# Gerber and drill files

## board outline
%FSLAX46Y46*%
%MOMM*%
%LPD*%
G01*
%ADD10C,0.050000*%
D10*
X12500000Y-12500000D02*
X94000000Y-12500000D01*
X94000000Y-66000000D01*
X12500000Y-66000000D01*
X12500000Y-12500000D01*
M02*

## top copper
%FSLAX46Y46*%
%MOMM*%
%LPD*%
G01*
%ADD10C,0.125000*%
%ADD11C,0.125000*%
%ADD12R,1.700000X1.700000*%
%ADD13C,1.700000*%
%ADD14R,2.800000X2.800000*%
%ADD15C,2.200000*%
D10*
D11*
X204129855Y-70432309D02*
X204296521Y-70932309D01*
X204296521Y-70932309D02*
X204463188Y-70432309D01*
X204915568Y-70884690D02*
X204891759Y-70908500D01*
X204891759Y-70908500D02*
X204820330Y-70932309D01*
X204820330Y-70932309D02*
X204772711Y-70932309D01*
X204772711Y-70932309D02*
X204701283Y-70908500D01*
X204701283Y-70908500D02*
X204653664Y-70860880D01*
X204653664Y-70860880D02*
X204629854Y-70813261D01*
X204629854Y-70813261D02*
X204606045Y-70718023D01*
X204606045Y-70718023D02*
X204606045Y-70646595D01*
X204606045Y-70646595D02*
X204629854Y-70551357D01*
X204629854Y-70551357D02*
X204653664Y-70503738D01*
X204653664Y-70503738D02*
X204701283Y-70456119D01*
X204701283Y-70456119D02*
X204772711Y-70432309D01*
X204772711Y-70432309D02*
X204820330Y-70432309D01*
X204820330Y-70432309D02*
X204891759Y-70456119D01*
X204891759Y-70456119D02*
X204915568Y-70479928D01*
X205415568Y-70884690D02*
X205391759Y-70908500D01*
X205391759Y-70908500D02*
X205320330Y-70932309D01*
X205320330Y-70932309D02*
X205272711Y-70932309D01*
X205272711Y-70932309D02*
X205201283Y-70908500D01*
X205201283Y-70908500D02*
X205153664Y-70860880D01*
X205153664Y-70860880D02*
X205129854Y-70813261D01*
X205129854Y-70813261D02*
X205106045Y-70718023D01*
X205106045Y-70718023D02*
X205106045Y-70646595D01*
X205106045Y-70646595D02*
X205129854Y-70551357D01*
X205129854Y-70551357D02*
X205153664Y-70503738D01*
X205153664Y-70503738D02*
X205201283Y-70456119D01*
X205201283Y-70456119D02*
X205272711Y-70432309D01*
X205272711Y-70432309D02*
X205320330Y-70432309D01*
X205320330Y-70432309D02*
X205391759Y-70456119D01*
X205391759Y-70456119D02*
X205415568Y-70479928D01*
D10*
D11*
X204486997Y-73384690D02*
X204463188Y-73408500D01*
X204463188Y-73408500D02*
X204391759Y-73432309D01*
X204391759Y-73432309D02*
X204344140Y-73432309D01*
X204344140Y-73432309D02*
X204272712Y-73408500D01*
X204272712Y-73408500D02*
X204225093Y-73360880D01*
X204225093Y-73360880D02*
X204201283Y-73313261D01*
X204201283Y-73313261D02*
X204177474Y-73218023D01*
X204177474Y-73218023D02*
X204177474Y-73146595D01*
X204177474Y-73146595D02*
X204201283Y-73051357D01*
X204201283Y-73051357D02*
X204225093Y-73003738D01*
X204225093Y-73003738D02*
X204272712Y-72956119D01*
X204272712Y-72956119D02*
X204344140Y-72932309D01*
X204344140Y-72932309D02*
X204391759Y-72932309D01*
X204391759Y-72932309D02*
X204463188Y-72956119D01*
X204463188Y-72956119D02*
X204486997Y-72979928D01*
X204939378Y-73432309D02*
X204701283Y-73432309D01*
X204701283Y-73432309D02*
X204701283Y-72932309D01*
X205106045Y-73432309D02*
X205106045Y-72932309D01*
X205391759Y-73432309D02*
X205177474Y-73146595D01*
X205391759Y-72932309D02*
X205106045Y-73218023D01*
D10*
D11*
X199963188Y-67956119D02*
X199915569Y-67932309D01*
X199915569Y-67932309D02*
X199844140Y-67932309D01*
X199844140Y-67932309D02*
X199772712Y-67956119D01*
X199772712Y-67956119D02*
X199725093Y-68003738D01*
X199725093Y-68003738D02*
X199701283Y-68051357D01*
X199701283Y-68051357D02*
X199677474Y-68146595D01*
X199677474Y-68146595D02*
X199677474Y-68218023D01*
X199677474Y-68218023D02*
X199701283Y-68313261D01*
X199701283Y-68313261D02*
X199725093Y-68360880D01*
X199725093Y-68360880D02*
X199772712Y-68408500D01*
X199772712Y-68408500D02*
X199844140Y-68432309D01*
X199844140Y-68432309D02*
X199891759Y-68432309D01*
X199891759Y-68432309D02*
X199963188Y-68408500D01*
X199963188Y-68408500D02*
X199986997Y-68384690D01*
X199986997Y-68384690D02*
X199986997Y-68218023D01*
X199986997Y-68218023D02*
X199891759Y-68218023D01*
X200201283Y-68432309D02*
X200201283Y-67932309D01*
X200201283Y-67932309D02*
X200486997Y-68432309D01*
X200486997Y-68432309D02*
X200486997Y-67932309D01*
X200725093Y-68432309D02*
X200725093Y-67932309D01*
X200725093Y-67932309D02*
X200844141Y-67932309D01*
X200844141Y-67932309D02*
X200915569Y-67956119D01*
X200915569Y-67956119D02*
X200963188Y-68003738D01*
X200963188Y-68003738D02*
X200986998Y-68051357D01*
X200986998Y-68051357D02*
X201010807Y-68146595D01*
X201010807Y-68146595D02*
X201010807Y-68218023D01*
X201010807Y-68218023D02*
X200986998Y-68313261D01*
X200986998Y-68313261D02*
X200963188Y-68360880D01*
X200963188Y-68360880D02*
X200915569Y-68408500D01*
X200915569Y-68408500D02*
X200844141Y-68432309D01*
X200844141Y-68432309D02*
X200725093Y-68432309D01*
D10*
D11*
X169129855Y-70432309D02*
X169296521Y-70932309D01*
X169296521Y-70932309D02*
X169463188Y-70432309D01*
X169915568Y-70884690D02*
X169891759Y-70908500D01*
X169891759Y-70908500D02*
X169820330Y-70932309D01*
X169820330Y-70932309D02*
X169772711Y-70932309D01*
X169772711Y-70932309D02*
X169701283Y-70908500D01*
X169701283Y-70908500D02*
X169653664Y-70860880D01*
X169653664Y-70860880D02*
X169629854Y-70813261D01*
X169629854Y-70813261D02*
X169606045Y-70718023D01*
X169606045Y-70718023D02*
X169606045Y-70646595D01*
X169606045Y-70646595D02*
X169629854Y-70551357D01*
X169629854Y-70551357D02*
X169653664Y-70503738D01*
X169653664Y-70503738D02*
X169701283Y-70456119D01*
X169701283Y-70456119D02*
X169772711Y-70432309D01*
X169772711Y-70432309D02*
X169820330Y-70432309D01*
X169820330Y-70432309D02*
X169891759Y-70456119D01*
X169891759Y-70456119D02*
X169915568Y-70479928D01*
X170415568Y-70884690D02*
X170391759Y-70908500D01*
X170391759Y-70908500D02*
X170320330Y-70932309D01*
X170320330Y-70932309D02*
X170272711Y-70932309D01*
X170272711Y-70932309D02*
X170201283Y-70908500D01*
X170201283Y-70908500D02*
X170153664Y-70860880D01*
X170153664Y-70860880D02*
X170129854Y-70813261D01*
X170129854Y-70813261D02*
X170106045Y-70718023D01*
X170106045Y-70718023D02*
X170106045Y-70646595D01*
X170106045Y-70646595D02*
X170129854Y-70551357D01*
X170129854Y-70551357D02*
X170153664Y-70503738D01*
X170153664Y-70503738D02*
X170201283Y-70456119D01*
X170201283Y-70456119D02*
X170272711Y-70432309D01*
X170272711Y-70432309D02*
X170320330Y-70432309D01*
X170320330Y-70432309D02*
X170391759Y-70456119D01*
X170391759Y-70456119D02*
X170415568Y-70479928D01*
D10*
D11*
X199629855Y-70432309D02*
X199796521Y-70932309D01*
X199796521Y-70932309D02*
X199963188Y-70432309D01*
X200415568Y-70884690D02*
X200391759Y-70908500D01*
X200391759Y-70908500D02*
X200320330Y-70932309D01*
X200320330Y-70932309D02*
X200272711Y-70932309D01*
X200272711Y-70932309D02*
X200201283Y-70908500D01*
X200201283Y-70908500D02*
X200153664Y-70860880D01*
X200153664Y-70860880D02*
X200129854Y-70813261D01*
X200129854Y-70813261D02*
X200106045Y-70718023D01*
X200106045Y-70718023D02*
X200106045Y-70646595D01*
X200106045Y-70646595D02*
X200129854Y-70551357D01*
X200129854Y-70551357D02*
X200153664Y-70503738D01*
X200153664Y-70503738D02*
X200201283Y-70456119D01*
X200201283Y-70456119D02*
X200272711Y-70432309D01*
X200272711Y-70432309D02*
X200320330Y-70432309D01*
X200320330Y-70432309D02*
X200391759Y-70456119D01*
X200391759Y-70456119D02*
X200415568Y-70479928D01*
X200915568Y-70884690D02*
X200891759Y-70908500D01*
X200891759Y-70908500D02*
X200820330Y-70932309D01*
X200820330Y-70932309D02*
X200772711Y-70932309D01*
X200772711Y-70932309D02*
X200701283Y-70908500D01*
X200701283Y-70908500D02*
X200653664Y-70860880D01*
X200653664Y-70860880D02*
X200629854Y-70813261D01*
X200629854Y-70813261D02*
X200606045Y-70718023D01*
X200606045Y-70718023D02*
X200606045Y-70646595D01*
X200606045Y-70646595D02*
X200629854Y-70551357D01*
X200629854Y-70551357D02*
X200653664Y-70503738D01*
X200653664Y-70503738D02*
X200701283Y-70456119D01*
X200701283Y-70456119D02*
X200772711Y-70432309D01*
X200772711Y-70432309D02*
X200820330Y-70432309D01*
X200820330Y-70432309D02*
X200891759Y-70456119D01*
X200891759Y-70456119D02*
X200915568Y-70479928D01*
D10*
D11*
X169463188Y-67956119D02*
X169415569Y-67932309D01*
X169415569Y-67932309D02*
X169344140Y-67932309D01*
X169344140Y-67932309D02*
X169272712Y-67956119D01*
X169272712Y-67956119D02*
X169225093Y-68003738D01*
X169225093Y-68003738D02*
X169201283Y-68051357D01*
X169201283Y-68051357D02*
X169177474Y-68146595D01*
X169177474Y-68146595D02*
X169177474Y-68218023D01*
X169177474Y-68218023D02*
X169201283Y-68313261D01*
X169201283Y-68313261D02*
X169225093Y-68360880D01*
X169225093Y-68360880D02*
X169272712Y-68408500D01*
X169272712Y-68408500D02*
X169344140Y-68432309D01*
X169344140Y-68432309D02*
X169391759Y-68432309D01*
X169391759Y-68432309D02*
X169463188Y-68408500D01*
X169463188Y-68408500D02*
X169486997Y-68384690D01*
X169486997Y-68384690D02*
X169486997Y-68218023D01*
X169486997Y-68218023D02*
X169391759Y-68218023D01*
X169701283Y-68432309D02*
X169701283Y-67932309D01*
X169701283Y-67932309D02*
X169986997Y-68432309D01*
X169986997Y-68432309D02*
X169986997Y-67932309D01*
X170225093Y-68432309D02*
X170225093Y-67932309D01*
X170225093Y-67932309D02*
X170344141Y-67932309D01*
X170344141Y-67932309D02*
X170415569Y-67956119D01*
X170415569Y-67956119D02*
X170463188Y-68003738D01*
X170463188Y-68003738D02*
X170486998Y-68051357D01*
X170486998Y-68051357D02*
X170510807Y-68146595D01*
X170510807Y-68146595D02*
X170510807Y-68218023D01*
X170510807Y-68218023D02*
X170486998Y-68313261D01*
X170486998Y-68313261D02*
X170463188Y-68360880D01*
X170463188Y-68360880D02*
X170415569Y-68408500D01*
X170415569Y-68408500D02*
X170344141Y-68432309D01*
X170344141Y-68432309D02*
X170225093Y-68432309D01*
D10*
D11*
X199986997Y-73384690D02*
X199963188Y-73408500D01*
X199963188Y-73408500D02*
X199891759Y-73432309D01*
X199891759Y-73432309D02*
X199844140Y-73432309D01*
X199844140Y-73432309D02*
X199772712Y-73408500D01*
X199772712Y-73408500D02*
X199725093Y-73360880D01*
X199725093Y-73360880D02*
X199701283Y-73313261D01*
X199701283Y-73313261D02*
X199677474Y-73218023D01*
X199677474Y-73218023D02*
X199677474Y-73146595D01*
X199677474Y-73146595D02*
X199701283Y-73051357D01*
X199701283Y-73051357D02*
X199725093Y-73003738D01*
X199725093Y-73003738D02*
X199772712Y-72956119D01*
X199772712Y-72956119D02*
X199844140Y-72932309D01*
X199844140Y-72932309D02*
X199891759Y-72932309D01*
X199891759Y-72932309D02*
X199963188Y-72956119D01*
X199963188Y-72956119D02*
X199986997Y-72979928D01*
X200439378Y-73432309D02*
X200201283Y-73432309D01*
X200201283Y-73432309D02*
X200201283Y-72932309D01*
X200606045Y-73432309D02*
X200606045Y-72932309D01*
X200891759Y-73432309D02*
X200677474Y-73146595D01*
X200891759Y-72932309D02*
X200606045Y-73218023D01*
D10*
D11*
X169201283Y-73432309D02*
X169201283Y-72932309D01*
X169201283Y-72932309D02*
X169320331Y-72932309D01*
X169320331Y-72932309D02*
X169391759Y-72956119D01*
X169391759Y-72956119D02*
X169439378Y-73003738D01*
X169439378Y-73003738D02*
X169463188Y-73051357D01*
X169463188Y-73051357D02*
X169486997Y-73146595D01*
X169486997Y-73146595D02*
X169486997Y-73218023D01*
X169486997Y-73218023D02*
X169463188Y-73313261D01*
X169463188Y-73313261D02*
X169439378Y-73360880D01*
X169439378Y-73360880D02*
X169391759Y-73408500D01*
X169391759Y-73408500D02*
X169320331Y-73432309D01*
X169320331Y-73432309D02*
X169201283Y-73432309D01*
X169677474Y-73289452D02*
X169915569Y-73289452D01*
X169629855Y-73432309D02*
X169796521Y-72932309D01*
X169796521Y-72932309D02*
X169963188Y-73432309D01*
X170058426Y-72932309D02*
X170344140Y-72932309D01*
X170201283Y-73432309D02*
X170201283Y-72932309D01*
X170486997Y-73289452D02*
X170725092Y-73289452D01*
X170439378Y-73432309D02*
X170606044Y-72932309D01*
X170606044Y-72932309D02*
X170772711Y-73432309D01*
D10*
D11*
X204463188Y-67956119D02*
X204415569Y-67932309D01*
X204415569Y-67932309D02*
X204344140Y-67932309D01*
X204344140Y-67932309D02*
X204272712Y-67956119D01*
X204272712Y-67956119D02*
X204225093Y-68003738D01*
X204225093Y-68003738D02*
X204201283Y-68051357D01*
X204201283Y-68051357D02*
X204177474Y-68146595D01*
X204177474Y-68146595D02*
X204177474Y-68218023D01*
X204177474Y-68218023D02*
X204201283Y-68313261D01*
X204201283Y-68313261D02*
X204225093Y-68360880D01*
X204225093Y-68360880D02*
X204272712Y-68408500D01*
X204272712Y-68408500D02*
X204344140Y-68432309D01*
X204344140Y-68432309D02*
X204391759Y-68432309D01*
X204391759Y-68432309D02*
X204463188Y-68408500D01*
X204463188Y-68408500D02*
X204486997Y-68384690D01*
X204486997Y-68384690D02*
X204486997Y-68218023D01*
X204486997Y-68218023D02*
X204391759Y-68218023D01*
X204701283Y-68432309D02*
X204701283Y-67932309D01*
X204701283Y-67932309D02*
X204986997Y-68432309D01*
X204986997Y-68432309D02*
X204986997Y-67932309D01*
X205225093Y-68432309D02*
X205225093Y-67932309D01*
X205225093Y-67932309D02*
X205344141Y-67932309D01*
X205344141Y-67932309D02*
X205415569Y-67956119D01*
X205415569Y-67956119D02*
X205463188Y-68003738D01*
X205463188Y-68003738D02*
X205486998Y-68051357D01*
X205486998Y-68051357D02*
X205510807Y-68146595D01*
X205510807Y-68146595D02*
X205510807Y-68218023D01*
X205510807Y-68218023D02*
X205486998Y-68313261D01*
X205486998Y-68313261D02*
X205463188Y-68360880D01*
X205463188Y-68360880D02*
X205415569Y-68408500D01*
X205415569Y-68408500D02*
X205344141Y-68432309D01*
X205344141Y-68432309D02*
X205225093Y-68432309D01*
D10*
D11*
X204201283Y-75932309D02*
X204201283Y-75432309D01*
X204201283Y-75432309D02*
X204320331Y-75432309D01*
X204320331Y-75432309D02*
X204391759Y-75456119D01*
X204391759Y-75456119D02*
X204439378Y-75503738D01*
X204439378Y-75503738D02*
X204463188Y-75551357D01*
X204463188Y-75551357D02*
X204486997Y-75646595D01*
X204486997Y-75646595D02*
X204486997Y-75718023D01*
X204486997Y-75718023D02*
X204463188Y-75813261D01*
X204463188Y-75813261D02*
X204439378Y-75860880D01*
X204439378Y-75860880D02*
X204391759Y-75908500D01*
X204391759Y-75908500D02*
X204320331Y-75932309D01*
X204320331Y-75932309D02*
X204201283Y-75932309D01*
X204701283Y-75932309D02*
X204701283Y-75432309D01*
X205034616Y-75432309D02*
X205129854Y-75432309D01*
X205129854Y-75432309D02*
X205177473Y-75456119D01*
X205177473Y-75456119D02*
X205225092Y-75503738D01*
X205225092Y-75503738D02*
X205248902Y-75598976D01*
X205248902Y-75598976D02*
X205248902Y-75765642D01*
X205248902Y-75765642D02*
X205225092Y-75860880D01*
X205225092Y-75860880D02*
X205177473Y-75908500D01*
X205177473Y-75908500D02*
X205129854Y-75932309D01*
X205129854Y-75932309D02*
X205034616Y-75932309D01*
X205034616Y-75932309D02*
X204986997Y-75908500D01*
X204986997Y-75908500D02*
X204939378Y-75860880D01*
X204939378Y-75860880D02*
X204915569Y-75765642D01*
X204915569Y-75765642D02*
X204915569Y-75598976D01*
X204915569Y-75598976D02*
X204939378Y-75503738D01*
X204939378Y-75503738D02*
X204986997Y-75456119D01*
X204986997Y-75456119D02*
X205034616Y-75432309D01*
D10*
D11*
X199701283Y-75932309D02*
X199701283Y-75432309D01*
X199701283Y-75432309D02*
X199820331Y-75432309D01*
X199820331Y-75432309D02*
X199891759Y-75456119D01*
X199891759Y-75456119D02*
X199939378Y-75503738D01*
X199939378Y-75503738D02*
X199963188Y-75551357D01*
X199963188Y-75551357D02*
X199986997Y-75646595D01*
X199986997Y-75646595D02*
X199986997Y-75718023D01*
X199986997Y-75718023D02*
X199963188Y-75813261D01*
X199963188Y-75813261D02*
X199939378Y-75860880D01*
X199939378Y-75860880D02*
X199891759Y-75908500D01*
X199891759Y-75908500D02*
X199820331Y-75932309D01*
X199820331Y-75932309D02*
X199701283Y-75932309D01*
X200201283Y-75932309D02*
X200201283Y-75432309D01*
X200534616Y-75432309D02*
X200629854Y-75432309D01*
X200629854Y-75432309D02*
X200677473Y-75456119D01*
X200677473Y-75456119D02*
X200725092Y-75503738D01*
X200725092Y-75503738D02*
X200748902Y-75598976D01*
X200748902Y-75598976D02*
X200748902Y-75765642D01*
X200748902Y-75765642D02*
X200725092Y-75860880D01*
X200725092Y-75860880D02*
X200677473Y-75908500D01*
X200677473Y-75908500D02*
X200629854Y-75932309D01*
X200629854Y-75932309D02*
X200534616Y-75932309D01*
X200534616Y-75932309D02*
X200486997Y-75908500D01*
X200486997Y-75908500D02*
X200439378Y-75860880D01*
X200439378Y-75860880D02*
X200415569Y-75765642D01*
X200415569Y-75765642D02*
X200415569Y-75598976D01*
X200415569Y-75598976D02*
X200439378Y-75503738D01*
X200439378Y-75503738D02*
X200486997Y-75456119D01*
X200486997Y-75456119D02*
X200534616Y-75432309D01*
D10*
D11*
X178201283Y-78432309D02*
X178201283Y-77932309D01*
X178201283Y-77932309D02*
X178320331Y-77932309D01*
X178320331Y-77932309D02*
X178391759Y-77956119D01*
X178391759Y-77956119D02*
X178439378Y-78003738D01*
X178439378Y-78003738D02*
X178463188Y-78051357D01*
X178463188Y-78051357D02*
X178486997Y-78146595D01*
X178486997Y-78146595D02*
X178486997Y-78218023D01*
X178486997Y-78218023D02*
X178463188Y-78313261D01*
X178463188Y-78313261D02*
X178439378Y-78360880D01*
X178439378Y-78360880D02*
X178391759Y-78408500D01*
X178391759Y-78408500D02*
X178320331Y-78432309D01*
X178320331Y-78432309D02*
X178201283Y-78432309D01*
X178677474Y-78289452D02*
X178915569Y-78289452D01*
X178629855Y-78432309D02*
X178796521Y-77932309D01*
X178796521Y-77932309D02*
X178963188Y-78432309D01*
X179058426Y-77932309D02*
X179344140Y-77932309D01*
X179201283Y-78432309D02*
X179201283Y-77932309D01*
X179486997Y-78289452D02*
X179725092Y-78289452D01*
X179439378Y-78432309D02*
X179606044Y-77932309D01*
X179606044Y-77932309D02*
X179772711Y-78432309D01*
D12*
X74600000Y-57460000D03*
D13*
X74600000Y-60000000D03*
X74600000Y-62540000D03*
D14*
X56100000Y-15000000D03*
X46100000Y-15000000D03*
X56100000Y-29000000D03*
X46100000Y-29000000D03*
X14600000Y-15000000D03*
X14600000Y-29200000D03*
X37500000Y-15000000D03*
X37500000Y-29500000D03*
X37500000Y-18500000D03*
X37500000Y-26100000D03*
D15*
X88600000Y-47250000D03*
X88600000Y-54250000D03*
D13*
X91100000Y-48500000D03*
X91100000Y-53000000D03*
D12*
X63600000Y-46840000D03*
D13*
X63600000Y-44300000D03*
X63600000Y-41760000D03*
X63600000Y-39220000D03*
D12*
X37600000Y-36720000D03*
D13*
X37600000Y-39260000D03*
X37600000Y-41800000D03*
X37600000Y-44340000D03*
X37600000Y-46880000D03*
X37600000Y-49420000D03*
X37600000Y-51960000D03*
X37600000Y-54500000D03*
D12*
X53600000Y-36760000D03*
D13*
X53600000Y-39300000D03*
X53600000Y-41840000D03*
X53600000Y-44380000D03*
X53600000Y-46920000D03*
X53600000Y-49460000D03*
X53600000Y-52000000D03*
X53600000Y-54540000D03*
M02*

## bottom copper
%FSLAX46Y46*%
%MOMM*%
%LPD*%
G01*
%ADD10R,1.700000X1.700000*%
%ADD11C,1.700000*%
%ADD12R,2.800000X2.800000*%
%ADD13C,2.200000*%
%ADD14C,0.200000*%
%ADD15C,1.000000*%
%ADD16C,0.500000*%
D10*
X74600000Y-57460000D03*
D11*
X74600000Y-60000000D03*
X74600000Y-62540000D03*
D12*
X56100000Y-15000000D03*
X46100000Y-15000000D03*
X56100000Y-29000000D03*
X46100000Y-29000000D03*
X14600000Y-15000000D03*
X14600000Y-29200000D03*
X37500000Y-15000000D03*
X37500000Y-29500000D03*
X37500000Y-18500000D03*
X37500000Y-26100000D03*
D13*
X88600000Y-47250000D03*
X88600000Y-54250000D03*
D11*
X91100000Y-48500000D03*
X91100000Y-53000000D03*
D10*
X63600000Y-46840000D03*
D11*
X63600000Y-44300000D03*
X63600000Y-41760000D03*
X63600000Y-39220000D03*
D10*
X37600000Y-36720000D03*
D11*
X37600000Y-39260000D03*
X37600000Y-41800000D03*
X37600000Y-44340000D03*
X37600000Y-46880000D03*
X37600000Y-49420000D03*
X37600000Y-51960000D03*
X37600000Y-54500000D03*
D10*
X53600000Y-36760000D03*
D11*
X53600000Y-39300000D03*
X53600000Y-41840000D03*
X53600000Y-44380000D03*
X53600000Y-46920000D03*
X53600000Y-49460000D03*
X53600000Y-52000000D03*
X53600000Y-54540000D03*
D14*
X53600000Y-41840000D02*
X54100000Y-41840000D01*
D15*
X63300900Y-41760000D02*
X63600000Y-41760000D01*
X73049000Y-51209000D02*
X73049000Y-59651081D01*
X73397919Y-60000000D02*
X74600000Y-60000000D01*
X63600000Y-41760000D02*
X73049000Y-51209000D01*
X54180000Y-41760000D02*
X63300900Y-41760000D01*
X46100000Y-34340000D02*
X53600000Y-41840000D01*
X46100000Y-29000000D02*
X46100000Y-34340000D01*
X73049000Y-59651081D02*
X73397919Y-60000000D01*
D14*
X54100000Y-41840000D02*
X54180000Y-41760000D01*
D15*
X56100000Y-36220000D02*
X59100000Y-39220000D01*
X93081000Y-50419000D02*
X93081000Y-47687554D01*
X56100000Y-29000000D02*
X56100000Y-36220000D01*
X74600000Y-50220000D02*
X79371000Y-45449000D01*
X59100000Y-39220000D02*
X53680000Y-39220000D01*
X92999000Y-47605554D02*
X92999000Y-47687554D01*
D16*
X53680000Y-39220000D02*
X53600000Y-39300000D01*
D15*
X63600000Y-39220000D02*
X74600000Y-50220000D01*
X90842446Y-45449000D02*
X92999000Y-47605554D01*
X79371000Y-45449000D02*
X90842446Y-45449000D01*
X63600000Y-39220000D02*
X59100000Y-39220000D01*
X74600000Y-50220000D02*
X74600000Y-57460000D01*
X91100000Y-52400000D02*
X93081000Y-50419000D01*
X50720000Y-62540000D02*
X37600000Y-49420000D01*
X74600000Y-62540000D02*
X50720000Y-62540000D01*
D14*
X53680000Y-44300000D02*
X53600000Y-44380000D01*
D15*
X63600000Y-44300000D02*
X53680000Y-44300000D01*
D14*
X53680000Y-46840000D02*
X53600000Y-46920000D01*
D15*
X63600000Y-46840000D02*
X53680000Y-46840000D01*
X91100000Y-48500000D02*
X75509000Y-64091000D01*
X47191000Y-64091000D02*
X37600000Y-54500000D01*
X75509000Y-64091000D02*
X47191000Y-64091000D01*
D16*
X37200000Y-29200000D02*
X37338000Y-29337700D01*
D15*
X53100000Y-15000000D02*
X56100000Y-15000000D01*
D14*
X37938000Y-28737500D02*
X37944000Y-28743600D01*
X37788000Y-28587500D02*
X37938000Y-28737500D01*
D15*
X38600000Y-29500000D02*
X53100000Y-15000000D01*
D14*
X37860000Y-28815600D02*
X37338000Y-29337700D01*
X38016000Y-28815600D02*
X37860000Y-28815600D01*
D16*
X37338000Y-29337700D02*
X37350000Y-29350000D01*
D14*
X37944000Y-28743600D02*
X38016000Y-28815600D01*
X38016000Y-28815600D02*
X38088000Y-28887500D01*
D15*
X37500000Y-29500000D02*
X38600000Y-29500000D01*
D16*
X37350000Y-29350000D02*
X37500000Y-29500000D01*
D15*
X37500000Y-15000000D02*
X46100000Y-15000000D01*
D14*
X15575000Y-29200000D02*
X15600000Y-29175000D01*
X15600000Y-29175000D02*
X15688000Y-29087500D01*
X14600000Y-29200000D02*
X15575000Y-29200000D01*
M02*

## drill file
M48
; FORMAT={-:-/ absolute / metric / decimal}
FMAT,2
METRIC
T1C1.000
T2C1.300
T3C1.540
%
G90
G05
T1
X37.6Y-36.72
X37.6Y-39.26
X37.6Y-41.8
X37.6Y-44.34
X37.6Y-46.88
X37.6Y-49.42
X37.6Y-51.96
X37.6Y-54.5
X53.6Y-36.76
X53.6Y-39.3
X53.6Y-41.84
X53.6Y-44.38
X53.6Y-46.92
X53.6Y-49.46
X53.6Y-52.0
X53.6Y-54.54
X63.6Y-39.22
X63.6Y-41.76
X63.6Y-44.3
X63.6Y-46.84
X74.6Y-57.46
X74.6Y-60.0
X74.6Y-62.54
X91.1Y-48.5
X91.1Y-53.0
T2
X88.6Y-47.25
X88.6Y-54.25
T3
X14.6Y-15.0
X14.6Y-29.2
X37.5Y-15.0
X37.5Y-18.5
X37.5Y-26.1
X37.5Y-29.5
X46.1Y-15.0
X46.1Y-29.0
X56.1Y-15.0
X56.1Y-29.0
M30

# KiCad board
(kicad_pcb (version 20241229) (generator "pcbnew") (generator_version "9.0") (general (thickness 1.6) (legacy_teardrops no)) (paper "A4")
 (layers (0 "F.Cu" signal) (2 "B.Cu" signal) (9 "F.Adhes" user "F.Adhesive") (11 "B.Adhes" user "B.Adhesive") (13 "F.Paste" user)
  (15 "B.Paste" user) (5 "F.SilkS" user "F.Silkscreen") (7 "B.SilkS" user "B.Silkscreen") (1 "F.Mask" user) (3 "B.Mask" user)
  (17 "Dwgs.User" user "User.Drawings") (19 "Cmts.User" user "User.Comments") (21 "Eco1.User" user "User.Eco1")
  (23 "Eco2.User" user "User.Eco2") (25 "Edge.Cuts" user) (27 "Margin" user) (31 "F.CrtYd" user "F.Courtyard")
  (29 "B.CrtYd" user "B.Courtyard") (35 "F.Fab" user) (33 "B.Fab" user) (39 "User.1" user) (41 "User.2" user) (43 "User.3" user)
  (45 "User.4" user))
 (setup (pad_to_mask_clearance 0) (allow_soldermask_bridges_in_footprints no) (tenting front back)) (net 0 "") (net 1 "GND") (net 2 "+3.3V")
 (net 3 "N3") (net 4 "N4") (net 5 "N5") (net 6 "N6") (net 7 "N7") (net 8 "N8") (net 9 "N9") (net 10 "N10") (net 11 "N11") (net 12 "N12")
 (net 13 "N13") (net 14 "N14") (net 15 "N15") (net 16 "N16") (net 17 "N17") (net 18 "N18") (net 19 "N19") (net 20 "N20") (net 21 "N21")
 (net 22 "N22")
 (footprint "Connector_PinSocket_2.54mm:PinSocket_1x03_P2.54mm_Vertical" (layer "F.Cu") (at 74.6 57.46)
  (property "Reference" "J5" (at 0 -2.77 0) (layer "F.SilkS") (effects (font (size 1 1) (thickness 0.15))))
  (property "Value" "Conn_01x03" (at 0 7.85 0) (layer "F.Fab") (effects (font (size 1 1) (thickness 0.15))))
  (pad "1" thru_hole rect (at 0 0) (size 1.7 1.7) (drill 1) (layers "*.Cu" "*.Mask") (remove_unused_layers no) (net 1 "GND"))
  (pad "2" thru_hole circle (at 0 2.54) (size 1.7 1.7) (drill 1) (layers "*.Cu" "*.Mask") (remove_unused_layers no) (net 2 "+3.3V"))
  (pad "3" thru_hole circle (at 0 5.08) (size 1.7 1.7) (drill 1) (layers "*.Cu" "*.Mask") (remove_unused_layers no) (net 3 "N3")))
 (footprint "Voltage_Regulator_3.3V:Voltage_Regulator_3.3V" (layer "F.Cu") (at 57.6 13.5 -90)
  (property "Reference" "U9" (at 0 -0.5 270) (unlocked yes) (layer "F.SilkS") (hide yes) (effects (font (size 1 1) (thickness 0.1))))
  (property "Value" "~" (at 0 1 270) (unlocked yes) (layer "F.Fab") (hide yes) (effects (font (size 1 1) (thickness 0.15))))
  (pad "1" thru_hole rect (at 1.5 1.5 180) (size 2.8 2.8) (drill 1.54) (layers "*.Cu" "*.Mask") (remove_unused_layers no) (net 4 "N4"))
  (pad "2" thru_hole rect (at 1.5 11.5 180) (size 2.8 2.8) (drill 1.54) (layers "*.Cu" "*.Mask") (remove_unused_layers no) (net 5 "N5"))
  (pad "3" thru_hole rect (at 15.5 1.5 180) (size 2.8 2.8) (drill 1.54) (layers "*.Cu" "*.Mask") (remove_unused_layers no) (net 1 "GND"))
  (pad "4" thru_hole rect (at 15.5 11.5 180) (size 2.8 2.8) (drill 1.54) (layers "*.Cu" "*.Mask") (remove_unused_layers no) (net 2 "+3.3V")))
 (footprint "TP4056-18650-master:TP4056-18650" (layer "F.Cu") (at 12.9 13.3)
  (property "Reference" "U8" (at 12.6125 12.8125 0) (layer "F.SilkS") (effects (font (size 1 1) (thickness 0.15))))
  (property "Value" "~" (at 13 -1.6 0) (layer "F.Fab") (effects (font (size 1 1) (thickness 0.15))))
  (pad "1" thru_hole rect (at 1.7 1.7) (size 2.8 2.8) (drill 1.54) (layers "*.Cu" "*.Mask") (remove_unused_layers no) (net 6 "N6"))
  (pad "2" thru_hole rect (at 1.7 15.9) (size 2.8 2.8) (drill 1.54) (layers "*.Cu" "*.Mask") (remove_unused_layers no) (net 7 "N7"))
  (pad "3" thru_hole rect (at 24.6 1.7) (size 2.8 2.8) (drill 1.54) (layers "*.Cu" "*.Mask") (remove_unused_layers no) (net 5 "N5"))
  (pad "4" thru_hole rect (at 24.6 16.2) (size 2.8 2.8) (drill 1.54) (layers "*.Cu" "*.Mask") (remove_unused_layers no) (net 4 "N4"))
  (pad "5" thru_hole rect (at 24.6 5.2) (size 2.8 2.8) (drill 1.54) (layers "*.Cu" "*.Mask") (remove_unused_layers no) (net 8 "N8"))
  (pad "6" thru_hole rect (at 24.6 12.8) (size 2.8 2.8) (drill 1.54) (layers "*.Cu" "*.Mask") (remove_unused_layers no) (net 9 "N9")))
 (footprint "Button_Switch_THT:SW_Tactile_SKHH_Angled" (layer "F.Cu") (at 91.1 48.5 -90)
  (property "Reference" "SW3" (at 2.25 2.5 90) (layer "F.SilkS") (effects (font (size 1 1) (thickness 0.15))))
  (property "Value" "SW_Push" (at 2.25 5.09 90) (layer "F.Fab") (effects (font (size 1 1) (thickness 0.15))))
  (pad "" thru_hole circle (at -1.25 2.5 90) (size 2.2 2.2) (drill 1.3) (layers "*.Cu" "*.Mask") (remove_unused_layers no))
  (pad "" thru_hole circle (at 5.75 2.5 90) (size 2.2 2.2) (drill 1.3) (layers "*.Cu" "*.Mask") (remove_unused_layers no))
  (pad "1" thru_hole circle (at 0 0 90) (size 1.7 1.7) (drill 1) (layers "*.Cu" "*.Mask") (remove_unused_layers no) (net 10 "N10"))
  (pad "2" thru_hole circle (at 4.5 0 90) (size 1.7 1.7) (drill 1) (layers "*.Cu" "*.Mask") (remove_unused_layers no) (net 1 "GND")))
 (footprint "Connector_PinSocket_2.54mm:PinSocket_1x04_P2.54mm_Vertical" (layer "F.Cu") (at 63.6 46.84 180)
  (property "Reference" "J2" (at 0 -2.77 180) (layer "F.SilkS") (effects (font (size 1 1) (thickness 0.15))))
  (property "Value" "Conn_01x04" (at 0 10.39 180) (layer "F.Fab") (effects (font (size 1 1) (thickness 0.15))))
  (pad "1" thru_hole rect (at 0 0 180) (size 1.7 1.7) (drill 1) (layers "*.Cu" "*.Mask") (remove_unused_layers no) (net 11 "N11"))
  (pad "2" thru_hole circle (at 0 2.54 180) (size 1.7 1.7) (drill 1) (layers "*.Cu" "*.Mask") (remove_unused_layers no) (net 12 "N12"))
  (pad "3" thru_hole circle (at 0 5.08 180) (size 1.7 1.7) (drill 1) (layers "*.Cu" "*.Mask") (remove_unused_layers no) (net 2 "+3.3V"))
  (pad "4" thru_hole circle (at 0 7.62 180) (size 1.7 1.7) (drill 1) (layers "*.Cu" "*.Mask") (remove_unused_layers no) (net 1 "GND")))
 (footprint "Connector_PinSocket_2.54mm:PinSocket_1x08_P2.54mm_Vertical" (layer "F.Cu") (at 37.6 36.72)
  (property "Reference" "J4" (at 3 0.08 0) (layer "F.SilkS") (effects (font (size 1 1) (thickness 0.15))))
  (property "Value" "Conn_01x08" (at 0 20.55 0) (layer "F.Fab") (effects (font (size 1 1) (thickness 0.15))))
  (pad "1" thru_hole rect (at 0 0) (size 1.7 1.7) (drill 1) (layers "*.Cu" "*.Mask") (remove_unused_layers no) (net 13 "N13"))
  (pad "2" thru_hole circle (at 0 2.54) (size 1.7 1.7) (drill 1) (layers "*.Cu" "*.Mask") (remove_unused_layers no) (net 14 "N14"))
  (pad "3" thru_hole circle (at 0 5.08) (size 1.7 1.7) (drill 1) (layers "*.Cu" "*.Mask") (remove_unused_layers no) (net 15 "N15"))
  (pad "4" thru_hole circle (at 0 7.62) (size 1.7 1.7) (drill 1) (layers "*.Cu" "*.Mask") (remove_unused_layers no) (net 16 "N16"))
  (pad "5" thru_hole circle (at 0 10.16) (size 1.7 1.7) (drill 1) (layers "*.Cu" "*.Mask") (remove_unused_layers no) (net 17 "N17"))
  (pad "6" thru_hole circle (at 0 12.7) (size 1.7 1.7) (drill 1) (layers "*.Cu" "*.Mask") (remove_unused_layers no) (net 3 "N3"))
  (pad "7" thru_hole circle (at 0 15.24) (size 1.7 1.7) (drill 1) (layers "*.Cu" "*.Mask") (remove_unused_layers no) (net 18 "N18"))
  (pad "8" thru_hole circle (at 0 17.78) (size 1.7 1.7) (drill 1) (layers "*.Cu" "*.Mask") (remove_unused_layers no) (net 10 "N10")))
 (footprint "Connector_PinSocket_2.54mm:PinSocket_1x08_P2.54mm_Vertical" (layer "F.Cu") (at 53.6 36.76)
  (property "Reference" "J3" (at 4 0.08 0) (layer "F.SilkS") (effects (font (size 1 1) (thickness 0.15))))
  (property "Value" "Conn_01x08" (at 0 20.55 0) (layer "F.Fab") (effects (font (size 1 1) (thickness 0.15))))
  (pad "1" thru_hole rect (at 0 0) (size 1.7 1.7) (drill 1) (layers "*.Cu" "*.Mask") (remove_unused_layers no) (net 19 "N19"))
  (pad "2" thru_hole circle (at 0 2.54) (size 1.7 1.7) (drill 1) (layers "*.Cu" "*.Mask") (remove_unused_layers no) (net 1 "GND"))
  (pad "3" thru_hole circle (at 0 5.08) (size 1.7 1.7) (drill 1) (layers "*.Cu" "*.Mask") (remove_unused_layers no) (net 2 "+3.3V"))
  (pad "4" thru_hole circle (at 0 7.62) (size 1.7 1.7) (drill 1) (layers "*.Cu" "*.Mask") (remove_unused_layers no) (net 12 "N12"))
  (pad "5" thru_hole circle (at 0 10.16) (size 1.7 1.7) (drill 1) (layers "*.Cu" "*.Mask") (remove_unused_layers no) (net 11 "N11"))
  (pad "6" thru_hole circle (at 0 12.7) (size 1.7 1.7) (drill 1) (layers "*.Cu" "*.Mask") (remove_unused_layers no) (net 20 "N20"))
  (pad "7" thru_hole circle (at 0 15.24) (size 1.7 1.7) (drill 1) (layers "*.Cu" "*.Mask") (remove_unused_layers no) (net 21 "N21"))
  (pad "8" thru_hole circle (at 0 17.78) (size 1.7 1.7) (drill 1) (layers "*.Cu" "*.Mask") (remove_unused_layers no) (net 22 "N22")))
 (gr_rect (start 12.5 12.5) (end 94 66) (stroke (width 0.05) (type default)) (fill no) (layer "Edge.Cuts"))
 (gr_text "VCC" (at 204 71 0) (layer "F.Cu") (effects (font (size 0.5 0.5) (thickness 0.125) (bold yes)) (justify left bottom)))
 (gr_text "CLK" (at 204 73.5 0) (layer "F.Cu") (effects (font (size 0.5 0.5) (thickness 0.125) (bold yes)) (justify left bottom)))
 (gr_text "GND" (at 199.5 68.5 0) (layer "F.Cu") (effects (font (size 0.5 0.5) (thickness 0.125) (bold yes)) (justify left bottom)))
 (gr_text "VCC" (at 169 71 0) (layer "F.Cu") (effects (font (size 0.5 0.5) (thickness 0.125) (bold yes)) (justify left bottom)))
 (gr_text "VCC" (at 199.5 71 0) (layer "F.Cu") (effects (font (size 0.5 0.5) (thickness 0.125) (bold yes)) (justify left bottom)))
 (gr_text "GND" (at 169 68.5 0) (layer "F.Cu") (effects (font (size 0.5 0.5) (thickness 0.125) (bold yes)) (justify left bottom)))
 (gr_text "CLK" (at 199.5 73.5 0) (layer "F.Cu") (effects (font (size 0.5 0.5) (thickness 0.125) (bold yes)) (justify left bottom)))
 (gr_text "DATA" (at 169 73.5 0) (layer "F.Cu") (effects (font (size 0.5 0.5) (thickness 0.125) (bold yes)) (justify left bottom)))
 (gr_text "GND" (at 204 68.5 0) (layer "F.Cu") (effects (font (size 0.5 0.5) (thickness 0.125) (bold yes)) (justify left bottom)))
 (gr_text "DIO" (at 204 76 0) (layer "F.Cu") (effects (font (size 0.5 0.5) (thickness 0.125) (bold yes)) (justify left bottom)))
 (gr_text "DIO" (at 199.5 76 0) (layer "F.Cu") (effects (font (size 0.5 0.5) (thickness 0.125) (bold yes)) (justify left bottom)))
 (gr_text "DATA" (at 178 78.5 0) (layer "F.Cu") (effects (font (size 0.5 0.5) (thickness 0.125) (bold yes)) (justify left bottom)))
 (segment (start 53.6 41.84) (end 54.1 41.84) (width 0.2) (layer "B.Cu") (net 2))
 (segment (start 63.3009 41.76) (end 63.6 41.76) (width 1) (layer "B.Cu") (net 2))
 (segment (start 73.049 51.209) (end 73.049 59.651081) (width 1) (layer "B.Cu") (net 2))
 (segment (start 73.397919 60) (end 74.6 60) (width 1) (layer "B.Cu") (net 2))
 (segment (start 63.6 41.76) (end 73.049 51.209) (width 1) (layer "B.Cu") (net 2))
 (segment (start 54.18 41.76) (end 63.3009 41.76) (width 1) (layer "B.Cu") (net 2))
 (segment (start 46.1 34.34) (end 53.6 41.84) (width 1) (layer "B.Cu") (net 2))
 (segment (start 46.1 29) (end 46.1 34.34) (width 1) (layer "B.Cu") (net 2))
 (segment (start 73.049 59.651081) (end 73.397919 60) (width 1) (layer "B.Cu") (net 2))
 (segment (start 54.1 41.84) (end 54.18 41.76) (width 0.2) (layer "B.Cu") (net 2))
 (segment (start 56.1 36.22) (end 59.1 39.22) (width 1) (layer "B.Cu") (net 1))
 (segment (start 93.081 50.419) (end 93.081 47.687554) (width 1) (layer "B.Cu") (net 1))
 (segment (start 56.1 29) (end 56.1 36.22) (width 1) (layer "B.Cu") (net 1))
 (segment (start 74.6 50.22) (end 79.371 45.449) (width 1) (layer "B.Cu") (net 1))
 (segment (start 59.1 39.22) (end 53.68 39.22) (width 1) (layer "B.Cu") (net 1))
 (segment (start 92.999 47.605554) (end 92.999 47.687554) (width 1) (layer "B.Cu") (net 1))
 (segment (start 53.68 39.22) (end 53.6 39.3) (width 0.5) (layer "B.Cu") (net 1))
 (segment (start 63.6 39.22) (end 74.6 50.22) (width 1) (layer "B.Cu") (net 1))
 (segment (start 90.842446 45.449) (end 92.999 47.605554) (width 1) (layer "B.Cu") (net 1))
 (segment (start 79.371 45.449) (end 90.842446 45.449) (width 1) (layer "B.Cu") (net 1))
 (segment (start 63.6 39.22) (end 59.1 39.22) (width 1) (layer "B.Cu") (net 1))
 (segment (start 74.6 50.22) (end 74.6 57.46) (width 1) (layer "B.Cu") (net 1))
 (segment (start 91.1 52.4) (end 93.081 50.419) (width 1) (layer "B.Cu") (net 1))
 (segment (start 50.72 62.54) (end 37.6 49.42) (width 1) (layer "B.Cu") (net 3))
 (segment (start 74.6 62.54) (end 50.72 62.54) (width 1) (layer "B.Cu") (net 3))
 (segment (start 53.68 44.3) (end 53.6 44.38) (width 0.2) (layer "B.Cu") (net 12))
 (segment (start 63.6 44.3) (end 53.68 44.3) (width 1) (layer "B.Cu") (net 12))
 (segment (start 53.68 46.84) (end 53.6 46.92) (width 0.2) (layer "B.Cu") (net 11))
 (segment (start 63.6 46.84) (end 53.68 46.84) (width 1) (layer "B.Cu") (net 11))
 (segment (start 91.1 48.5) (end 75.509 64.091) (width 1) (layer "B.Cu") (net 10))
 (segment (start 47.191 64.091) (end 37.6 54.5) (width 1) (layer "B.Cu") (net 10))
 (segment (start 75.509 64.091) (end 47.191 64.091) (width 1) (layer "B.Cu") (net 10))
 (segment (start 37.2 29.2) (end 37.338 29.3377) (width 0.5) (layer "B.Cu") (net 4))
 (segment (start 53.1 15) (end 56.1 15) (width 1) (layer "B.Cu") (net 4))
 (segment (start 37.938 28.7375) (end 37.944 28.7436) (width 0.2) (layer "B.Cu") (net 4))
 (segment (start 37.788 28.5875) (end 37.938 28.7375) (width 0.2) (layer "B.Cu") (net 4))
 (segment (start 38.6 29.5) (end 53.1 15) (width 1) (layer "B.Cu") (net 4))
 (segment (start 37.86 28.8156) (end 37.338 29.3377) (width 0.2) (layer "B.Cu") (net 4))
 (segment (start 38.016 28.8156) (end 37.86 28.8156) (width 0.2) (layer "B.Cu") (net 4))
 (segment (start 37.338 29.3377) (end 37.35 29.35) (width 0.5) (layer "B.Cu") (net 4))
 (segment (start 37.944 28.7436) (end 38.016 28.8156) (width 0.2) (layer "B.Cu") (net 4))
 (segment (start 38.016 28.8156) (end 38.088 28.8875) (width 0.2) (layer "B.Cu") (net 4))
 (segment (start 37.5 29.5) (end 38.6 29.5) (width 1) (layer "B.Cu") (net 4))
 (segment (start 37.35 29.35) (end 37.5 29.5) (width 0.5) (layer "B.Cu") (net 4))
 (segment (start 37.5 15) (end 46.1 15) (width 1) (layer "B.Cu") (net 5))
 (segment (start 15.575 29.2) (end 15.6 29.175) (width 0.2) (layer "B.Cu") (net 7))
 (segment (start 15.6 29.175) (end 15.688 29.0875) (width 0.2) (layer "B.Cu") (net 7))
 (segment (start 14.6 29.2) (end 15.575 29.2) (width 0.2) (layer "B.Cu") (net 7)))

